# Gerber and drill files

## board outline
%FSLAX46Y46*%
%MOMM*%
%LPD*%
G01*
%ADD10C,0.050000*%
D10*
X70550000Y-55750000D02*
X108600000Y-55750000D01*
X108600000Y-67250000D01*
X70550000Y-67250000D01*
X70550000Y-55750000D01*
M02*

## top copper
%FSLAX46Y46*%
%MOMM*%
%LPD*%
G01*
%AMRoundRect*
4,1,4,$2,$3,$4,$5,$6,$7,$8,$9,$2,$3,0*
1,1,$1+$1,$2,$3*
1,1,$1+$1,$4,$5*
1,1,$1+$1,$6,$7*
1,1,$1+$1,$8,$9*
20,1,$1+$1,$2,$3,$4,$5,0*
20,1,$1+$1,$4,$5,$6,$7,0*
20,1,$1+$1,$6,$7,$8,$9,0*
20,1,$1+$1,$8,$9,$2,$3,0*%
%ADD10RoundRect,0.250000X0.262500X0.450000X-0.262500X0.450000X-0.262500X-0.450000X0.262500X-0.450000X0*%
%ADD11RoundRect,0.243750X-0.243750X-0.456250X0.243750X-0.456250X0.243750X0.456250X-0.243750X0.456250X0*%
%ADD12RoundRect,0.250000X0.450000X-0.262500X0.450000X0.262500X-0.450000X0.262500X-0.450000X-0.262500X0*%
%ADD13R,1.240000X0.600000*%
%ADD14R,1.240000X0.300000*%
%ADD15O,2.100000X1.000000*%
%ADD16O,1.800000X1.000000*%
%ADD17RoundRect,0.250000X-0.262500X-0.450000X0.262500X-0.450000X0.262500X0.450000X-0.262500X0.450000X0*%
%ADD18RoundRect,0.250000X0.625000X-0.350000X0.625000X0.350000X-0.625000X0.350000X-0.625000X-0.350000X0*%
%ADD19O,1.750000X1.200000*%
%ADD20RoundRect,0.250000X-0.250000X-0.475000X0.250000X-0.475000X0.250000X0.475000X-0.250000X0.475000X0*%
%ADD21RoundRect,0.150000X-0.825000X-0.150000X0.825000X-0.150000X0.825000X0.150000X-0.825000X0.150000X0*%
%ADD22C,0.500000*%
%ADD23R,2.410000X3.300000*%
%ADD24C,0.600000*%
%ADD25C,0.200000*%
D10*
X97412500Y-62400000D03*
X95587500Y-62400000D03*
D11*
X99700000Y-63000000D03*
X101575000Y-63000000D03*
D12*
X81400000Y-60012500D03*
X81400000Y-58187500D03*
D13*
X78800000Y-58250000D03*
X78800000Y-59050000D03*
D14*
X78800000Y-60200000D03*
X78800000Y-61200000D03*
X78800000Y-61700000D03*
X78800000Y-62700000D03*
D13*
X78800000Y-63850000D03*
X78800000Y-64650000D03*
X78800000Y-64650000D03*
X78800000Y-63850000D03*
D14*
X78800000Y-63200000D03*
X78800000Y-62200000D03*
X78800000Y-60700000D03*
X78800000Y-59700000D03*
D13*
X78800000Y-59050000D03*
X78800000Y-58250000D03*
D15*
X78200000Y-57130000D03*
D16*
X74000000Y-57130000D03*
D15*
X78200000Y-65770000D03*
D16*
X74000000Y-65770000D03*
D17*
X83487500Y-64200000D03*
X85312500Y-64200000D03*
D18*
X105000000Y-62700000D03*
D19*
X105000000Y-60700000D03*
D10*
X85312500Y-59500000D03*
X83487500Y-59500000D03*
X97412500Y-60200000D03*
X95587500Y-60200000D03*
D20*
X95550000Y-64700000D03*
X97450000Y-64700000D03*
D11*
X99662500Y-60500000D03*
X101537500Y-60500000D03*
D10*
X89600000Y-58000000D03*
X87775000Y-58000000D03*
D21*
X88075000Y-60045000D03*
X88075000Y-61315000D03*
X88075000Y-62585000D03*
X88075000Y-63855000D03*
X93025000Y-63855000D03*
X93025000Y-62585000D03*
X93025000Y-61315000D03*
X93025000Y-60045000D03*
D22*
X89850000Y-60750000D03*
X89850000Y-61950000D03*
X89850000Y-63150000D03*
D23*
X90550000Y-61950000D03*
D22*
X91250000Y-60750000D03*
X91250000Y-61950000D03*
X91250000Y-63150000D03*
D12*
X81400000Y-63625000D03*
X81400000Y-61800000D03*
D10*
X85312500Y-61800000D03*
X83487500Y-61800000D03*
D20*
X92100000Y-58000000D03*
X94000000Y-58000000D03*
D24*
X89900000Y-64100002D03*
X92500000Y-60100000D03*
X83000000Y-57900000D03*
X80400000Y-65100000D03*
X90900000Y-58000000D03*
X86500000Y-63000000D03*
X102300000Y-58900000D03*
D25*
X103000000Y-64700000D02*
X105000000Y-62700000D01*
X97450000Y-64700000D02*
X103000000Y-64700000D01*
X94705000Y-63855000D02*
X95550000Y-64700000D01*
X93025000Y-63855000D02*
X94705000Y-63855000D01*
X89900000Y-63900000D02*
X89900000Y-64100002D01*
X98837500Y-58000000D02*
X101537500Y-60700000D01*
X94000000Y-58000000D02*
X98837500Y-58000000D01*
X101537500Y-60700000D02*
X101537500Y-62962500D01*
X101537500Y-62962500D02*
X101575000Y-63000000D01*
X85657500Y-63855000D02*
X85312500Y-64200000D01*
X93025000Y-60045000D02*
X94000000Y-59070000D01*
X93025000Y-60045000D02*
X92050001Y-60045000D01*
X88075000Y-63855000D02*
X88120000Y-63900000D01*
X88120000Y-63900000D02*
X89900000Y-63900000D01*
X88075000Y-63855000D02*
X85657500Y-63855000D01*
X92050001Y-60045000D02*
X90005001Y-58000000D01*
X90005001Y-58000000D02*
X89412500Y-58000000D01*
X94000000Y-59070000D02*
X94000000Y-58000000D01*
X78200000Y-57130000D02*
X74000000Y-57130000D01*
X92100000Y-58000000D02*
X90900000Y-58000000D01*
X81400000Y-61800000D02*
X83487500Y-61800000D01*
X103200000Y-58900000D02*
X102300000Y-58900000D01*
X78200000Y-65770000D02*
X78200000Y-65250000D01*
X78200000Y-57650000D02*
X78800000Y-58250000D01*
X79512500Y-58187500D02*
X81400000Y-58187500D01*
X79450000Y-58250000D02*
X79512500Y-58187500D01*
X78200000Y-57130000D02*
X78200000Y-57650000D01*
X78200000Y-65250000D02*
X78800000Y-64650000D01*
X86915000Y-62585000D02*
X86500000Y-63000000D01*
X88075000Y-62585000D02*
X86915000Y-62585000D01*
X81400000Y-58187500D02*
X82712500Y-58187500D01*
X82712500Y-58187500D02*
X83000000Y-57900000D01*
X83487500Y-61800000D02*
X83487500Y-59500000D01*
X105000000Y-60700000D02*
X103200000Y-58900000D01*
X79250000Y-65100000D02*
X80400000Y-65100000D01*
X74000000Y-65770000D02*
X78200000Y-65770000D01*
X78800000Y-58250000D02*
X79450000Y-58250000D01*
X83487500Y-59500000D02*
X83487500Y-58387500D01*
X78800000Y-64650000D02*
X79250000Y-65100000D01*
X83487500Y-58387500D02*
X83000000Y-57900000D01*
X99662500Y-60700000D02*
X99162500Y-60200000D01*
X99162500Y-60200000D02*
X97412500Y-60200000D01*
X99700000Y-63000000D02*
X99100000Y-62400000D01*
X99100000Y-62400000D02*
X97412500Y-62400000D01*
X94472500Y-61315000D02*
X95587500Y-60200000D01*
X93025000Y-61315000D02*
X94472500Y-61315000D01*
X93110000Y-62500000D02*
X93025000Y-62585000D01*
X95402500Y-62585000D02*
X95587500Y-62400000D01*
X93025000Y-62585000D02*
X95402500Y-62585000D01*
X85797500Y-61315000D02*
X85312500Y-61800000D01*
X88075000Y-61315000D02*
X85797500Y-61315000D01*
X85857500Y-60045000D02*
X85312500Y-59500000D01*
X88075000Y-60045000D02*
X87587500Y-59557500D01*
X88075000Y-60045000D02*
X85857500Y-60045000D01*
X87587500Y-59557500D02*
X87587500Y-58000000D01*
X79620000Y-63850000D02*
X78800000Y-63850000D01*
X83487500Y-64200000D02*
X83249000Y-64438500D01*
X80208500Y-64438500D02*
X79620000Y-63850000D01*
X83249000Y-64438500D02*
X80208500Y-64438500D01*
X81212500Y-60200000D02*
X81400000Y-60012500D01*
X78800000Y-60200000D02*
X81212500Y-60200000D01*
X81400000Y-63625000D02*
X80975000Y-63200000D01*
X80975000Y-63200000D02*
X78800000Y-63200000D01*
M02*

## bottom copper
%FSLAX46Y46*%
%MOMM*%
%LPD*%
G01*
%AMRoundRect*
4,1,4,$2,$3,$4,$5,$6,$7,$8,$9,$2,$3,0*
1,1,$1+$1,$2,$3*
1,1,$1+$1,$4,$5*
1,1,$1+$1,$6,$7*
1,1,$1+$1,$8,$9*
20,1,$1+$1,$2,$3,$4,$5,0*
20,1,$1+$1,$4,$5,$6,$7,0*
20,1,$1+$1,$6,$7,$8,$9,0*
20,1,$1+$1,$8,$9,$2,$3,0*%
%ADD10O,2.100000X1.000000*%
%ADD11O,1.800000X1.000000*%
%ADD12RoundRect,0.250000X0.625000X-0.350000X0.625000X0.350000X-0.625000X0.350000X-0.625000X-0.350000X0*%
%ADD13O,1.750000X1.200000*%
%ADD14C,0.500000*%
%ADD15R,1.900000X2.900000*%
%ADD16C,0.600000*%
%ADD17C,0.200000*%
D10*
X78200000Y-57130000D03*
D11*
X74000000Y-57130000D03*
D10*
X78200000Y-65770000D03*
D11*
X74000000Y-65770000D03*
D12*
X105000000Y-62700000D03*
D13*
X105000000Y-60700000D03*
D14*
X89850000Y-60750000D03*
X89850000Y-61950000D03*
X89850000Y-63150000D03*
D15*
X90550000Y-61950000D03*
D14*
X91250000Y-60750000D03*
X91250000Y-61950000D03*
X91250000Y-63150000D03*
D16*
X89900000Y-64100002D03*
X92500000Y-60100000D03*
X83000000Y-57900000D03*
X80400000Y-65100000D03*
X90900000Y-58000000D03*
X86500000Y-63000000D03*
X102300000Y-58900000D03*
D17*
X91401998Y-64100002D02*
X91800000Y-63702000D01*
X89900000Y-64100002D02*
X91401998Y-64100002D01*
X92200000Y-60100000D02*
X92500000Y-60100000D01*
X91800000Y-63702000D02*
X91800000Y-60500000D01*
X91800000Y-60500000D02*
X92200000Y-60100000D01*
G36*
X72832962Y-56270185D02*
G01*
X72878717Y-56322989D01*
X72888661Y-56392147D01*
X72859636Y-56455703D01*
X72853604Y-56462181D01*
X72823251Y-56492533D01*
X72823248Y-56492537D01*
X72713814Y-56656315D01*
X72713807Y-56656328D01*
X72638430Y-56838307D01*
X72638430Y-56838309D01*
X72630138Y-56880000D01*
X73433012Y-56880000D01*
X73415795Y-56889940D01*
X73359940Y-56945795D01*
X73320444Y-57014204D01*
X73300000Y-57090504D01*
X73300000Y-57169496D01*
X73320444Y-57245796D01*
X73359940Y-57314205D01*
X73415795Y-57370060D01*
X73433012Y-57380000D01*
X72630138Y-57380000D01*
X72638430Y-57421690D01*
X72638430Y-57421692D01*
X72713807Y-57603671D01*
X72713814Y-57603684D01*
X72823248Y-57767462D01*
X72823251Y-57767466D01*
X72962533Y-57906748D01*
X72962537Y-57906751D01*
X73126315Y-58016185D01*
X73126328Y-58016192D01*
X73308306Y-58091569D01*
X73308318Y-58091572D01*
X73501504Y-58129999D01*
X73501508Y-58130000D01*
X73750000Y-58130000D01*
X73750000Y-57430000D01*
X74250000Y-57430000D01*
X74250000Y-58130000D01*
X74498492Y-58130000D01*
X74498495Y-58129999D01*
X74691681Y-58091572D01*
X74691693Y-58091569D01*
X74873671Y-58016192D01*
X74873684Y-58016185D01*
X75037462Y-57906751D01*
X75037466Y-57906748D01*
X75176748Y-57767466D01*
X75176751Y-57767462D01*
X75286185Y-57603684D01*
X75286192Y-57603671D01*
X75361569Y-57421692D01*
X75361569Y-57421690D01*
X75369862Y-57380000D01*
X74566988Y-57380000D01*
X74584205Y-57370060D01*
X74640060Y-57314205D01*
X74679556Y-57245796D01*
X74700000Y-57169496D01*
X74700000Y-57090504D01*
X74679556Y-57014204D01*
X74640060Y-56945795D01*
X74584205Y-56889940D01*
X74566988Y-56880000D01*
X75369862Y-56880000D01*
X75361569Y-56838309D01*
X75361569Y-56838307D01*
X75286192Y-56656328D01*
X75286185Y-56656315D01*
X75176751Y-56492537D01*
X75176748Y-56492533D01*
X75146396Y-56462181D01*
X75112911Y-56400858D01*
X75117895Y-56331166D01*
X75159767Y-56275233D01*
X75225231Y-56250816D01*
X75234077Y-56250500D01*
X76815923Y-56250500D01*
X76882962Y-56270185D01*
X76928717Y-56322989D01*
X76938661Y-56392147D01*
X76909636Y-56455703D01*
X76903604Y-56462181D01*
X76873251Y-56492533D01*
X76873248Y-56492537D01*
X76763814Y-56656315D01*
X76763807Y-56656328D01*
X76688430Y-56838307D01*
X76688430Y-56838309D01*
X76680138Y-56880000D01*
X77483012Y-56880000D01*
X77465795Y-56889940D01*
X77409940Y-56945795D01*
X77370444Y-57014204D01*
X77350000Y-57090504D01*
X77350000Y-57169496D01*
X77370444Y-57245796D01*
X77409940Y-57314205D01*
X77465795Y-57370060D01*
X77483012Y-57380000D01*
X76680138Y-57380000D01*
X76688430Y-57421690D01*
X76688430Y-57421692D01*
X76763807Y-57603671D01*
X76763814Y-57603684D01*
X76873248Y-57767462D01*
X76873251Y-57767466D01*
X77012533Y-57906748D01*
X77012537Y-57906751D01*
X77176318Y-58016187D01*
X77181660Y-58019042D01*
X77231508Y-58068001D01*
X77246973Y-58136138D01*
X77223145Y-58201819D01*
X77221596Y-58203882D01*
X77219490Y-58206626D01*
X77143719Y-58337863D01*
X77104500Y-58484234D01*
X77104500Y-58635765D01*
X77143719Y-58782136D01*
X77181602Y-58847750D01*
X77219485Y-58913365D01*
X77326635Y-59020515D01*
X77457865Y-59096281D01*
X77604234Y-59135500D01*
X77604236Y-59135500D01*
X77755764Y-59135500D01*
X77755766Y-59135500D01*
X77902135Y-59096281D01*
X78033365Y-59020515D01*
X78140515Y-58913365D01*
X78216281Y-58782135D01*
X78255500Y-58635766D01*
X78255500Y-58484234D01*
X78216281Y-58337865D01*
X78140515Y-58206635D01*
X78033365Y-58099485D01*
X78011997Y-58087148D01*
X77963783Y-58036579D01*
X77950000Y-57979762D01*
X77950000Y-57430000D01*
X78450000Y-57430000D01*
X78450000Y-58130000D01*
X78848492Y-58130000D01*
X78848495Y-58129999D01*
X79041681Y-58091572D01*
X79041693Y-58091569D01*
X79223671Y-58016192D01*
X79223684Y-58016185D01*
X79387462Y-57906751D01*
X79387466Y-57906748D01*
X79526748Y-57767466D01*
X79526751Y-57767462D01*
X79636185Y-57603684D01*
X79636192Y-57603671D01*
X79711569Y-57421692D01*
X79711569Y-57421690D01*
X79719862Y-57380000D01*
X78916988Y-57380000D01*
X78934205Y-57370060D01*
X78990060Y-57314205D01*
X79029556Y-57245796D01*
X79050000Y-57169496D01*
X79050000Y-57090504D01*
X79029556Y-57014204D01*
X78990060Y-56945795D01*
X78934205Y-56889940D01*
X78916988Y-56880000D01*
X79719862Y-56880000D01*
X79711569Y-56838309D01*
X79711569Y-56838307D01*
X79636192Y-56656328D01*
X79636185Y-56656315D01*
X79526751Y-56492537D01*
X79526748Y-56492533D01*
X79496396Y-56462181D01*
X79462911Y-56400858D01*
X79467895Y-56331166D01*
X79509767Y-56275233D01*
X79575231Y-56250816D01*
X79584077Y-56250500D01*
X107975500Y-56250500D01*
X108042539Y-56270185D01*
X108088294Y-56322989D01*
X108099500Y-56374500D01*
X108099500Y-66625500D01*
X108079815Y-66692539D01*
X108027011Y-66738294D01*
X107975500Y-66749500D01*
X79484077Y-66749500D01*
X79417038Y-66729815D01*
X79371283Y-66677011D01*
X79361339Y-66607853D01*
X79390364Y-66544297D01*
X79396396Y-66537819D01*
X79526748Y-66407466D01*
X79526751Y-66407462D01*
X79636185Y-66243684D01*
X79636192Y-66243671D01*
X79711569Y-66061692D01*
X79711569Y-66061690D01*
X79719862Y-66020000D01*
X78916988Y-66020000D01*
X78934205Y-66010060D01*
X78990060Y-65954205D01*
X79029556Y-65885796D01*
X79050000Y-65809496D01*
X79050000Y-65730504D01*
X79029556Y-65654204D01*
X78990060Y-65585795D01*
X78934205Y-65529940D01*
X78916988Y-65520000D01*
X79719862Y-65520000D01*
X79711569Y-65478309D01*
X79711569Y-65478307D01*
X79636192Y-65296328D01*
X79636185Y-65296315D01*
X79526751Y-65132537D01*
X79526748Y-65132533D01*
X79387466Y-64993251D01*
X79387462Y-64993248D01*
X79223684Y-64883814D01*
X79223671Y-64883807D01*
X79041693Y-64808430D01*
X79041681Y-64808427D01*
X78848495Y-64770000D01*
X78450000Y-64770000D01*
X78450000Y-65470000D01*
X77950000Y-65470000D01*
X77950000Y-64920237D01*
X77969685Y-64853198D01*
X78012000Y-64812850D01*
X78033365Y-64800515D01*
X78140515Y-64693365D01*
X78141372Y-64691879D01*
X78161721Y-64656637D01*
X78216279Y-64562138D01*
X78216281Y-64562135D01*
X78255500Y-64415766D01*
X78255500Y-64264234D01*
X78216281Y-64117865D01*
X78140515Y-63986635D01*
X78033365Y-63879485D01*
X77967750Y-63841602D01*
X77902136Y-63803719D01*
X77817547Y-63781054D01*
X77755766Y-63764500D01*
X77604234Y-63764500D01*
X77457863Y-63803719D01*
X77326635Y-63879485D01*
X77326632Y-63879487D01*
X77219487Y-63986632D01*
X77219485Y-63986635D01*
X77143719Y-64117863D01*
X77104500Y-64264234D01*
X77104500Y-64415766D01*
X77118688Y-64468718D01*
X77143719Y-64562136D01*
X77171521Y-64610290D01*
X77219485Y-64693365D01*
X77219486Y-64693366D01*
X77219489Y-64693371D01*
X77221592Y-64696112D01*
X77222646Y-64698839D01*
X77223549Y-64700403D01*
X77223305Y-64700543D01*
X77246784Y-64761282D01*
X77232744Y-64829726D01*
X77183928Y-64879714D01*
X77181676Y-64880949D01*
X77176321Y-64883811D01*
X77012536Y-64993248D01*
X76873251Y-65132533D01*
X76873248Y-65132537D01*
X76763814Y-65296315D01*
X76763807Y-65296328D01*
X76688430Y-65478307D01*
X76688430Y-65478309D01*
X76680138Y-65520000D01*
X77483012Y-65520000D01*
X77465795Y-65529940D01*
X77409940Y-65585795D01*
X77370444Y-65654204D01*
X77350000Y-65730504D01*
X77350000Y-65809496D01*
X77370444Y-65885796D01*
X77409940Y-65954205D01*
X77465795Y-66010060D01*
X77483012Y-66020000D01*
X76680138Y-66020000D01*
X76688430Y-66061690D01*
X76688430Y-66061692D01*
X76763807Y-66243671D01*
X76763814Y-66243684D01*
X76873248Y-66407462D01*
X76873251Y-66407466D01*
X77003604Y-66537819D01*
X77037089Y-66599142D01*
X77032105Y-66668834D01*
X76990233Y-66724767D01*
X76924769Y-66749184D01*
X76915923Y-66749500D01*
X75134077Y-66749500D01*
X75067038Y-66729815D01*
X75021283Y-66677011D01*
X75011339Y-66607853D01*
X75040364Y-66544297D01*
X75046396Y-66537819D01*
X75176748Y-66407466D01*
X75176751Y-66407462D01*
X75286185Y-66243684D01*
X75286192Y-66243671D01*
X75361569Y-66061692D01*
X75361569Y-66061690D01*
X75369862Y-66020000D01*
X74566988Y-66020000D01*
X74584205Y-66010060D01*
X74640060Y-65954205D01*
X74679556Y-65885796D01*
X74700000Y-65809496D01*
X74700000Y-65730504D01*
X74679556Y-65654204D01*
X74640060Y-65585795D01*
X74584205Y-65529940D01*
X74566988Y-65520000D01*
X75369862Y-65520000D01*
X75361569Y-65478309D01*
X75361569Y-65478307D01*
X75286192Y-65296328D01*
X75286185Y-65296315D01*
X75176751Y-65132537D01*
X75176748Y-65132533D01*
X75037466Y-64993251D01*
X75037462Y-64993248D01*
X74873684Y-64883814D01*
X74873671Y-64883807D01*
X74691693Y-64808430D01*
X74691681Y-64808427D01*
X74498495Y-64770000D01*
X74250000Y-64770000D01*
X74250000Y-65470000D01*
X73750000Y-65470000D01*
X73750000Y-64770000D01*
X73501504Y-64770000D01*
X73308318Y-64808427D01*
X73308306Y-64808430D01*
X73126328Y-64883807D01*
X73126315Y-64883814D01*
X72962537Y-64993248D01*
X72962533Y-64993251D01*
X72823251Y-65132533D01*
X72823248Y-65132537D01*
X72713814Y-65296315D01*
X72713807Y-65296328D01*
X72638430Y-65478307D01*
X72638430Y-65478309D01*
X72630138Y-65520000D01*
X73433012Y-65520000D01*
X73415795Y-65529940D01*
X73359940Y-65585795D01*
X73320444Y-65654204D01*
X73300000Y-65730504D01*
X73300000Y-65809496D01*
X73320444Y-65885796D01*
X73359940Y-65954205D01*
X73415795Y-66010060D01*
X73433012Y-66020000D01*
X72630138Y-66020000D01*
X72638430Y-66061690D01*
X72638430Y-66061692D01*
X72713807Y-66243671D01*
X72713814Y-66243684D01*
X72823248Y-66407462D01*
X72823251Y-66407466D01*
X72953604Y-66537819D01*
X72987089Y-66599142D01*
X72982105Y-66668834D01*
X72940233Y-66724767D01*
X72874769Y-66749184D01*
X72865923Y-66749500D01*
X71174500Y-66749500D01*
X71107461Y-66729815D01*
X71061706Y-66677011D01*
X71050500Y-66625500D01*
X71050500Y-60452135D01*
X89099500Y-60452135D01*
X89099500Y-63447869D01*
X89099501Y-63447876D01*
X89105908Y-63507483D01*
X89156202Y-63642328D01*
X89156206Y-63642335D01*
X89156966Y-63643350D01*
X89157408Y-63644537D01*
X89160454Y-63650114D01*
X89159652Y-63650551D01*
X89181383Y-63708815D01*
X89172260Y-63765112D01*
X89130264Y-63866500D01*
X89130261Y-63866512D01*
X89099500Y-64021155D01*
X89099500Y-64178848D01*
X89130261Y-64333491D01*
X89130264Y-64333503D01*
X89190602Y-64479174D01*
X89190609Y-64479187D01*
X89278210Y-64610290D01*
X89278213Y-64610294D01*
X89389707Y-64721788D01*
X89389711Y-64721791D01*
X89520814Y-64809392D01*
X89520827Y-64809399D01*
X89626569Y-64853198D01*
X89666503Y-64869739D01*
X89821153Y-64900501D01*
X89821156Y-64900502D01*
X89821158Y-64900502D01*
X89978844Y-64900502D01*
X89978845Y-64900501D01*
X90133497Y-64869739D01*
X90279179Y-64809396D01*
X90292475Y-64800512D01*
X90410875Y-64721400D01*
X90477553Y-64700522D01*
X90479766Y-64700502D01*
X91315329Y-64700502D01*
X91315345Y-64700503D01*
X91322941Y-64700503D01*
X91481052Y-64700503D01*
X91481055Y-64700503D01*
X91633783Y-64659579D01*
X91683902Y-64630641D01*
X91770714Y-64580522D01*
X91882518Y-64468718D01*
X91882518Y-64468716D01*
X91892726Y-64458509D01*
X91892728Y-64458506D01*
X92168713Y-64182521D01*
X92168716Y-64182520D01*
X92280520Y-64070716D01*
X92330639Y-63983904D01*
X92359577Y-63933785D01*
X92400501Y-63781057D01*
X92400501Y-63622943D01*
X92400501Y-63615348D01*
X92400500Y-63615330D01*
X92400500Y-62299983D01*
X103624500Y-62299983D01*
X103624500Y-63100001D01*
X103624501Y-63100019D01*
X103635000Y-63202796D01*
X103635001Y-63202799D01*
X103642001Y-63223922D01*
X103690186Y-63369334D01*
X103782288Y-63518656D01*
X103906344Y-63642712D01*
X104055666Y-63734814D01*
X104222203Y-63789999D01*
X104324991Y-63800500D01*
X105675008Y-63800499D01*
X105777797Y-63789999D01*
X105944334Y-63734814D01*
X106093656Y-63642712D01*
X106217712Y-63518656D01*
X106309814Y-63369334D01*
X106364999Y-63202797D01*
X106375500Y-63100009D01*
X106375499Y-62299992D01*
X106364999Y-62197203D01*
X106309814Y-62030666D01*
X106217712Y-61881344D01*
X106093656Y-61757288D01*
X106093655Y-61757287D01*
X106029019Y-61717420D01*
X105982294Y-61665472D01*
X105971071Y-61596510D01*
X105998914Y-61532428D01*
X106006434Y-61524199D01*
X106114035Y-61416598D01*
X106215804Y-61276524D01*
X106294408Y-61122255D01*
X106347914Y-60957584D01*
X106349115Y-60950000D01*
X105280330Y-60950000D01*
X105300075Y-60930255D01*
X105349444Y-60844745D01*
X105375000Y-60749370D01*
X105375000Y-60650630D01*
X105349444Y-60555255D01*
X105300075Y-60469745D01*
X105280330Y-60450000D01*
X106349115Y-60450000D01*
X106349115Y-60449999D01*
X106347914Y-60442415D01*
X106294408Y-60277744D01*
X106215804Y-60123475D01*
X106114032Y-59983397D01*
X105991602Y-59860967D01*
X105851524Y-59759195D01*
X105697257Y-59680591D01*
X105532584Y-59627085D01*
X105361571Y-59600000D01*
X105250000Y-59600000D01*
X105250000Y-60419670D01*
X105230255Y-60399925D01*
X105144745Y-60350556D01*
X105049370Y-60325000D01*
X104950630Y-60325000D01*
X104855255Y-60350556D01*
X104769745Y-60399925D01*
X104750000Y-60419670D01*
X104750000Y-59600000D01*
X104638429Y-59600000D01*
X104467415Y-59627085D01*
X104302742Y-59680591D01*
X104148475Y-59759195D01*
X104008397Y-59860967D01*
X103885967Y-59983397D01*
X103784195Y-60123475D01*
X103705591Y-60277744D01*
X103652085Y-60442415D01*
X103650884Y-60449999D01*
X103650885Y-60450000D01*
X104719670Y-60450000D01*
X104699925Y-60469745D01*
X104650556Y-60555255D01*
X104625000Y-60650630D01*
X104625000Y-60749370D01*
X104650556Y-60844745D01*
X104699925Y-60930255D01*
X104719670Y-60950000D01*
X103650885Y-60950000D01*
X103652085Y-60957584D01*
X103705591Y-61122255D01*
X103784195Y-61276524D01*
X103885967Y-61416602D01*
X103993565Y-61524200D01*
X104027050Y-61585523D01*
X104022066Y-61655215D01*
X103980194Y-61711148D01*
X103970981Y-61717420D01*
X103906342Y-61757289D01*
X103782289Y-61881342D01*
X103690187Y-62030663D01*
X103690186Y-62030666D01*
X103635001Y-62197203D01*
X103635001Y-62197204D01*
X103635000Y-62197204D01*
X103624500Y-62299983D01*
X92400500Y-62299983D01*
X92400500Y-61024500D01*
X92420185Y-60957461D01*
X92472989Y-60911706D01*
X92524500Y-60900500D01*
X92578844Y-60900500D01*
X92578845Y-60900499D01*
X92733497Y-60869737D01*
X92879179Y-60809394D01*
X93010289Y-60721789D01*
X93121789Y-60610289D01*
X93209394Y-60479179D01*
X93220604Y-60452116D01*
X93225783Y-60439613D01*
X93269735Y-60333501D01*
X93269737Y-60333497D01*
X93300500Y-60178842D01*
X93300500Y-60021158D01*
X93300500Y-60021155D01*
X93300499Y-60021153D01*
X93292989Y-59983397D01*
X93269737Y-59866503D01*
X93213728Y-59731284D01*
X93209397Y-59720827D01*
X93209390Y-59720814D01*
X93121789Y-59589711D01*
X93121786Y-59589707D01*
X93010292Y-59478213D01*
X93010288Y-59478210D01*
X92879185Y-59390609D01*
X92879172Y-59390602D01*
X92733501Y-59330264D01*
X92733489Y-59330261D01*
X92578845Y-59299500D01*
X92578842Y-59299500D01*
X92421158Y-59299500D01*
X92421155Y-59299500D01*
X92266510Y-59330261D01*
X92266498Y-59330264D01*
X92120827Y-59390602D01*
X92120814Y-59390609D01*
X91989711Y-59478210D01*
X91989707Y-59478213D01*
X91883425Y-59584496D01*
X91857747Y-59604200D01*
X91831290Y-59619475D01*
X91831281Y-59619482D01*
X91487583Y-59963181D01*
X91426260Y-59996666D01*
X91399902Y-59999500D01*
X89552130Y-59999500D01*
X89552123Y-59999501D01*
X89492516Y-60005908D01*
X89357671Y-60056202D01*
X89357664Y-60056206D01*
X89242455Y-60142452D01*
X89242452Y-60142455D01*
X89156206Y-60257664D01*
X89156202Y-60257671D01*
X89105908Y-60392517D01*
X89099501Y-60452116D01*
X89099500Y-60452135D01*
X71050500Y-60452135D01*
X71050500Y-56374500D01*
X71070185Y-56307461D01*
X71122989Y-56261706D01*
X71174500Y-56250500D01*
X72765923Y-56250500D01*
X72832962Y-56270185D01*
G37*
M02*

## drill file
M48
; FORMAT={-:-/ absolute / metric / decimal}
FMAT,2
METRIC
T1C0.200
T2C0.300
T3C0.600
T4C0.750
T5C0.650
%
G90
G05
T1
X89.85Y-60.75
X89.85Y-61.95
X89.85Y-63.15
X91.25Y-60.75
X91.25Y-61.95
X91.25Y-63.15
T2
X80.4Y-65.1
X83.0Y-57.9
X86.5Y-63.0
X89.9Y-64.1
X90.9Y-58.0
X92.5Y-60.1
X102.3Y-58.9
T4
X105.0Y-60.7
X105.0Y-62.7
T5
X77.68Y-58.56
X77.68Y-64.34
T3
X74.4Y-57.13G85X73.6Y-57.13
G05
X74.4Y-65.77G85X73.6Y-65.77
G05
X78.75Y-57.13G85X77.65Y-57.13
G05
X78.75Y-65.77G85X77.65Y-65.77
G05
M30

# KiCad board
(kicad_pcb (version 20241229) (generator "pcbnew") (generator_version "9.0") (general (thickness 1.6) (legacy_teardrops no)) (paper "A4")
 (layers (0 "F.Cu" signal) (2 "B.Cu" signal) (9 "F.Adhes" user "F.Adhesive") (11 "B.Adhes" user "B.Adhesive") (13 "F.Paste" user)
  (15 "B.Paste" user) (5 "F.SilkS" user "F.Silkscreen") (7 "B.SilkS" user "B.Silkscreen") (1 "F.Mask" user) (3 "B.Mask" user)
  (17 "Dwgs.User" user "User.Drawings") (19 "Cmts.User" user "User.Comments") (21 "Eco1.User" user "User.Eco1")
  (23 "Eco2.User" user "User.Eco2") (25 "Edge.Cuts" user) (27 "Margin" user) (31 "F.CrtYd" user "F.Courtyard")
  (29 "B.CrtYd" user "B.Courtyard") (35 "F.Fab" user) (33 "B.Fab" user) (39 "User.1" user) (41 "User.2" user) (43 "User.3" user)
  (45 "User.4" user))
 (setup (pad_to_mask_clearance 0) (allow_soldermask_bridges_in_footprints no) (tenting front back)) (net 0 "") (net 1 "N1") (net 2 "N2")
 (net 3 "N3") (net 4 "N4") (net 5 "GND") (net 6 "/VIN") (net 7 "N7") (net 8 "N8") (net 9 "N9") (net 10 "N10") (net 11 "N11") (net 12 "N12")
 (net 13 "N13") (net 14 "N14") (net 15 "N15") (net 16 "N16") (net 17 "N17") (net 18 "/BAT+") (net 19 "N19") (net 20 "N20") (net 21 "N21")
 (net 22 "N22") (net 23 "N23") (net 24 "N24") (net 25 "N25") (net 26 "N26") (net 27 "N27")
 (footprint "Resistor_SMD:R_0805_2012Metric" (layer "F.Cu") (at 96.5 62.4 180)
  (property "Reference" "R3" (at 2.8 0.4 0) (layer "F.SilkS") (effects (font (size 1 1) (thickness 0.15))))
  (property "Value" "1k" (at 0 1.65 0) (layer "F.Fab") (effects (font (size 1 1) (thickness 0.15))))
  (pad "1" smd roundrect (at -0.9125 0 180) (size 1.025 1.4) (layers "F.Cu" "F.Mask" "F.Paste") (roundrect_rratio 0.243902) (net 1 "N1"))
  (pad "2" smd roundrect (at 0.9125 0 180) (size 1.025 1.4) (layers "F.Cu" "F.Mask" "F.Paste") (roundrect_rratio 0.243902) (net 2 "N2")))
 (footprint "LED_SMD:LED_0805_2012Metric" (layer "F.Cu") (at 100.6375 63)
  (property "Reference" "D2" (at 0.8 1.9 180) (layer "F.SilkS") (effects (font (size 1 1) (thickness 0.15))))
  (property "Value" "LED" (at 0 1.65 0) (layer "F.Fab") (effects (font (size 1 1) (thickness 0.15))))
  (pad "1" smd roundrect (at -0.9375 0) (size 0.975 1.4) (layers "F.Cu" "F.Mask" "F.Paste") (roundrect_rratio 0.25) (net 1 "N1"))
  (pad "2" smd roundrect (at 0.9375 0) (size 0.975 1.4) (layers "F.Cu" "F.Mask" "F.Paste") (roundrect_rratio 0.25) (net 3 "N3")))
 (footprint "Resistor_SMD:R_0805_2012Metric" (layer "F.Cu") (at 81.4 59.1 90)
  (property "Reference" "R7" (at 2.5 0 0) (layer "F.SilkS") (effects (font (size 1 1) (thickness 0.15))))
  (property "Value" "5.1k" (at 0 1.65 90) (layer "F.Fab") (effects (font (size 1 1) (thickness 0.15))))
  (pad "1" smd roundrect (at -0.9125 0 90) (size 1.025 1.4) (layers "F.Cu" "F.Mask" "F.Paste") (roundrect_rratio 0.243902) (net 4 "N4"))
  (pad "2" smd roundrect (at 0.9125 0 90) (size 1.025 1.4) (layers "F.Cu" "F.Mask" "F.Paste") (roundrect_rratio 0.243902) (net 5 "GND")))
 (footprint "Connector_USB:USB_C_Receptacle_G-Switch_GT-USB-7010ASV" (layer "F.Cu") (at 75.075 61.45 -90)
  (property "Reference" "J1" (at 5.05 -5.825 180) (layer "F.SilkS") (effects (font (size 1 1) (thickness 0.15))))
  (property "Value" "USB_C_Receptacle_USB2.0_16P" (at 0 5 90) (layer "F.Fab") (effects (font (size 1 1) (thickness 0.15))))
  (pad "" np_thru_hole circle (at -2.89 -2.605 270) (size 0.65 0.65) (drill 0.65) (layers "*.Cu" "*.Mask"))
  (pad "" np_thru_hole circle (at 2.89 -2.605 270) (size 0.65 0.65) (drill 0.65) (layers "*.Cu" "*.Mask"))
  (pad "A1" smd rect (at -3.2 -3.725 270) (size 0.6 1.24) (layers "F.Cu" "F.Mask" "F.Paste") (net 5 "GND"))
  (pad "A4" smd rect (at -2.4 -3.725 270) (size 0.6 1.24) (layers "F.Cu" "F.Mask" "F.Paste") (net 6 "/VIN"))
  (pad "A5" smd rect (at -1.25 -3.725 270) (size 0.3 1.24) (layers "F.Cu" "F.Mask" "F.Paste") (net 4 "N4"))
  (pad "A6" smd rect (at -0.25 -3.725 270) (size 0.3 1.24) (layers "F.Cu" "F.Mask" "F.Paste") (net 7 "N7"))
  (pad "A7" smd rect (at 0.25 -3.725 270) (size 0.3 1.24) (layers "F.Cu" "F.Mask" "F.Paste") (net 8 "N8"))
  (pad "A8" smd rect (at 1.25 -3.725 270) (size 0.3 1.24) (layers "F.Cu" "F.Mask" "F.Paste") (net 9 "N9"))
  (pad "A9" smd rect (at 2.4 -3.725 270) (size 0.6 1.24) (layers "F.Cu" "F.Mask" "F.Paste") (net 6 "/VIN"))
  (pad "A12" smd rect (at 3.2 -3.725 270) (size 0.6 1.24) (layers "F.Cu" "F.Mask" "F.Paste") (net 5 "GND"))
  (pad "B1" smd rect (at 3.2 -3.725 270) (size 0.6 1.24) (layers "F.Cu" "F.Mask" "F.Paste") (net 5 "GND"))
  (pad "B4" smd rect (at 2.4 -3.725 270) (size 0.6 1.24) (layers "F.Cu" "F.Mask" "F.Paste") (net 6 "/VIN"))
  (pad "B5" smd rect (at 1.75 -3.725 270) (size 0.3 1.24) (layers "F.Cu" "F.Mask" "F.Paste") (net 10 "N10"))
  (pad "B6" smd rect (at 0.75 -3.725 270) (size 0.3 1.24) (layers "F.Cu" "F.Mask" "F.Paste") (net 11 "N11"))
  (pad "B7" smd rect (at -0.75 -3.725 270) (size 0.3 1.24) (layers "F.Cu" "F.Mask" "F.Paste") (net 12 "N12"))
  (pad "B8" smd rect (at -1.75 -3.725 270) (size 0.3 1.24) (layers "F.Cu" "F.Mask" "F.Paste") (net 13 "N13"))
  (pad "B9" smd rect (at -2.4 -3.725 270) (size 0.6 1.24) (layers "F.Cu" "F.Mask" "F.Paste") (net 6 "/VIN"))
  (pad "B12" smd rect (at -3.2 -3.725 270) (size 0.6 1.24) (layers "F.Cu" "F.Mask" "F.Paste") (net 5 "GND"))
  (pad "S1" thru_hole oval (at -4.32 -3.125 270) (size 1 2.1) (drill oval 0.6 1.7) (layers "*.Cu" "*.Mask") (remove_unused_layers no)
   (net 5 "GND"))
  (pad "S1" thru_hole oval (at -4.32 1.075 270) (size 1 1.8) (drill oval 0.6 1.4) (layers "*.Cu" "*.Mask") (remove_unused_layers no)
   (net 5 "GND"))
  (pad "S1" thru_hole oval (at 4.32 -3.125 270) (size 1 2.1) (drill oval 0.6 1.7) (layers "*.Cu" "*.Mask") (remove_unused_layers no)
   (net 5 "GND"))
  (pad "S1" thru_hole oval (at 4.32 1.075 270) (size 1 1.8) (drill oval 0.6 1.4) (layers "*.Cu" "*.Mask") (remove_unused_layers no)
   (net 5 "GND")))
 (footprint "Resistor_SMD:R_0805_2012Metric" (layer "F.Cu") (at 84.4 64.2)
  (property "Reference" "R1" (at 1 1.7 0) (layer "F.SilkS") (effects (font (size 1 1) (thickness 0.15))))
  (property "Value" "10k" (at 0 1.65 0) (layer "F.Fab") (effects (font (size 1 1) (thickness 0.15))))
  (pad "1" smd roundrect (at -0.9125 0) (size 1.025 1.4) (layers "F.Cu" "F.Mask" "F.Paste") (roundrect_rratio 0.243902) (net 6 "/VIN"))
  (pad "2" smd roundrect (at 0.9125 0) (size 1.025 1.4) (layers "F.Cu" "F.Mask" "F.Paste") (roundrect_rratio 0.243902) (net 3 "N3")))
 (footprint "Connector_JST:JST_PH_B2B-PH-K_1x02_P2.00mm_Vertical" (layer "F.Cu") (at 105 62.7 90)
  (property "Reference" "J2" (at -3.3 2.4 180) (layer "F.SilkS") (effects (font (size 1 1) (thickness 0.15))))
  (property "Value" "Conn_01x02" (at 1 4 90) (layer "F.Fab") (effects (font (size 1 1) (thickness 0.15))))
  (pad "1" thru_hole roundrect (at 0 0 90) (size 1.2 1.75) (drill 0.75) (layers "*.Cu" "*.Mask") (remove_unused_layers no)
   (roundrect_rratio 0.208333) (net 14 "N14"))
  (pad "2" thru_hole oval (at 2 0 90) (size 1.2 1.75) (drill 0.75) (layers "*.Cu" "*.Mask") (remove_unused_layers no) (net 5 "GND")))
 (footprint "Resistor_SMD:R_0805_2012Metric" (layer "F.Cu") (at 84.4 59.5 180)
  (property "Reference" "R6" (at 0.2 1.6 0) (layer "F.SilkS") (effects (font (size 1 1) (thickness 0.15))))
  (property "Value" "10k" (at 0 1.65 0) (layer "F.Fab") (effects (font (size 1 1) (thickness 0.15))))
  (pad "1" smd roundrect (at -0.9125 0 180) (size 1.025 1.4) (layers "F.Cu" "F.Mask" "F.Paste") (roundrect_rratio 0.243902) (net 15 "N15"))
  (pad "2" smd roundrect (at 0.9125 0 180) (size 1.025 1.4) (layers "F.Cu" "F.Mask" "F.Paste") (roundrect_rratio 0.243902) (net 5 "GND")))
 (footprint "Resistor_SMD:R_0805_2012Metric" (layer "F.Cu") (at 96.5 60.2 180)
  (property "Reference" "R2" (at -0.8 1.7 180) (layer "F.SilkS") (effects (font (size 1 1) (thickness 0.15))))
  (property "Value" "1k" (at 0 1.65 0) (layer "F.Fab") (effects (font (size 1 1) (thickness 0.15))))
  (pad "1" smd roundrect (at -0.9125 0 180) (size 1.025 1.4) (layers "F.Cu" "F.Mask" "F.Paste") (roundrect_rratio 0.243902) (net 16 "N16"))
  (pad "2" smd roundrect (at 0.9125 0 180) (size 1.025 1.4) (layers "F.Cu" "F.Mask" "F.Paste") (roundrect_rratio 0.243902) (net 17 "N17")))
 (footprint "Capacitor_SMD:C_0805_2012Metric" (layer "F.Cu") (at 96.5 64.7)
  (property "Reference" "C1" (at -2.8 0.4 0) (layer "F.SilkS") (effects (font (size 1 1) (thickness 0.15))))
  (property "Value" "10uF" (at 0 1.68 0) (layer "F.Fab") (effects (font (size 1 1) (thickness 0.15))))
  (pad "1" smd roundrect (at -0.95 0) (size 1 1.45) (layers "F.Cu" "F.Mask" "F.Paste") (roundrect_rratio 0.25) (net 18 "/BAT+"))
  (pad "2" smd roundrect (at 0.95 0) (size 1 1.45) (layers "F.Cu" "F.Mask" "F.Paste") (roundrect_rratio 0.25) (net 14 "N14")))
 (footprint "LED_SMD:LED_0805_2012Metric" (layer "F.Cu") (at 100.6 60.5)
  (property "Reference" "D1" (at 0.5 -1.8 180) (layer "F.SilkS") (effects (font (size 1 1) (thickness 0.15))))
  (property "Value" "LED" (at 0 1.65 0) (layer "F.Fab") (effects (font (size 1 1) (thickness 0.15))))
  (pad "1" smd roundrect (at -0.9375 0) (size 0.975 1.4) (layers "F.Cu" "F.Mask" "F.Paste") (roundrect_rratio 0.25) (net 16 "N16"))
  (pad "2" smd roundrect (at 0.9375 0) (size 0.975 1.4) (layers "F.Cu" "F.Mask" "F.Paste") (roundrect_rratio 0.25) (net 3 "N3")))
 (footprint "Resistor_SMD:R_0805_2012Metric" (layer "F.Cu") (at 88.6875 58 180)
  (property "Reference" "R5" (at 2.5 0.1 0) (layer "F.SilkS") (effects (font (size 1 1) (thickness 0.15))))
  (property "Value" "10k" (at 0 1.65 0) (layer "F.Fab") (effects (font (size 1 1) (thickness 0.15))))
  (pad "1" smd roundrect (at -0.9125 0 180) (size 1.025 1.4) (layers "F.Cu" "F.Mask" "F.Paste") (roundrect_rratio 0.243902) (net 3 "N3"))
  (pad "2" smd roundrect (at 0.9125 0 180) (size 1.025 1.4) (layers "F.Cu" "F.Mask" "F.Paste") (roundrect_rratio 0.243902) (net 15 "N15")))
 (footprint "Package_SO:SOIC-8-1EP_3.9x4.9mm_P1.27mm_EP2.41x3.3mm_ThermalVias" (layer "F.Cu") (at 90.55 61.95)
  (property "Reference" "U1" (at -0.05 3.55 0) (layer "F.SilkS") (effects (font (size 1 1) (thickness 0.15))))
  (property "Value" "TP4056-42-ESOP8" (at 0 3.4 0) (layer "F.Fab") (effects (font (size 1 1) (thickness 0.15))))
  (pad "" smd roundrect (at -0.6 -0.825) (size 1.01 1.38) (layers "F.Paste") (roundrect_rratio 0.247525))
  (pad "" smd roundrect (at -0.6 0.825) (size 1.01 1.38) (layers "F.Paste") (roundrect_rratio 0.247525))
  (pad "" smd roundrect (at 0.6 -0.825) (size 1.01 1.38) (layers "F.Paste") (roundrect_rratio 0.247525))
  (pad "" smd roundrect (at 0.6 0.825) (size 1.01 1.38) (layers "F.Paste") (roundrect_rratio 0.247525))
  (pad "1" smd roundrect (at -2.475 -1.905) (size 1.95 0.6) (layers "F.Cu" "F.Mask" "F.Paste") (roundrect_rratio 0.25) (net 15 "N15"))
  (pad "2" smd roundrect (at -2.475 -0.635) (size 1.95 0.6) (layers "F.Cu" "F.Mask" "F.Paste") (roundrect_rratio 0.25) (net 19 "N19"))
  (pad "3" smd roundrect (at -2.475 0.635) (size 1.95 0.6) (layers "F.Cu" "F.Mask" "F.Paste") (roundrect_rratio 0.25) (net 5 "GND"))
  (pad "4" smd roundrect (at -2.475 1.905) (size 1.95 0.6) (layers "F.Cu" "F.Mask" "F.Paste") (roundrect_rratio 0.25) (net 3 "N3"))
  (pad "5" smd roundrect (at 2.475 1.905) (size 1.95 0.6) (layers "F.Cu" "F.Mask" "F.Paste") (roundrect_rratio 0.25) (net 18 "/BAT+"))
  (pad "6" smd roundrect (at 2.475 0.635) (size 1.95 0.6) (layers "F.Cu" "F.Mask" "F.Paste") (roundrect_rratio 0.25) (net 2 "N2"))
  (pad "7" smd roundrect (at 2.475 -0.635) (size 1.95 0.6) (layers "F.Cu" "F.Mask" "F.Paste") (roundrect_rratio 0.25) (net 17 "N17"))
  (pad "8" smd roundrect (at 2.475 -1.905) (size 1.95 0.6) (layers "F.Cu" "F.Mask" "F.Paste") (roundrect_rratio 0.25) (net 3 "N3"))
  (pad "9" thru_hole circle (at -0.7 -1.2) (size 0.5 0.5) (drill 0.2) (layers "*.Cu") (remove_unused_layers no) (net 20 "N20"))
  (pad "9" thru_hole circle (at -0.7 0) (size 0.5 0.5) (drill 0.2) (layers "*.Cu") (remove_unused_layers no) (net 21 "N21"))
  (pad "9" thru_hole circle (at -0.7 1.2) (size 0.5 0.5) (drill 0.2) (layers "*.Cu") (remove_unused_layers no) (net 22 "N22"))
  (pad "9" smd rect (at 0 0) (size 1.9 2.9) (layers "B.Cu") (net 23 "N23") (zone_connect 2))
  (pad "9" smd rect (at 0 0) (size 2.41 3.3) (layers "F.Cu" "F.Mask") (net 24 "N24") (zone_connect 2))
  (pad "9" thru_hole circle (at 0.7 -1.2) (size 0.5 0.5) (drill 0.2) (layers "*.Cu") (remove_unused_layers no) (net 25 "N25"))
  (pad "9" thru_hole circle (at 0.7 0) (size 0.5 0.5) (drill 0.2) (layers "*.Cu") (remove_unused_layers no) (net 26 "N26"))
  (pad "9" thru_hole circle (at 0.7 1.2) (size 0.5 0.5) (drill 0.2) (layers "*.Cu") (remove_unused_layers no) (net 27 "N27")))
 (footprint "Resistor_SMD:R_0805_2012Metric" (layer "F.Cu") (at 81.4 62.7125 90)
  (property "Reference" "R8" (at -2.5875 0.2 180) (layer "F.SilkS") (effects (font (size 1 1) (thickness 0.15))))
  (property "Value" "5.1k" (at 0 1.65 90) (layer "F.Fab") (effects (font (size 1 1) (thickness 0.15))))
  (pad "1" smd roundrect (at -0.9125 0 90) (size 1.025 1.4) (layers "F.Cu" "F.Mask" "F.Paste") (roundrect_rratio 0.243902) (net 10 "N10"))
  (pad "2" smd roundrect (at 0.9125 0 90) (size 1.025 1.4) (layers "F.Cu" "F.Mask" "F.Paste") (roundrect_rratio 0.243902) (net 5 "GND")))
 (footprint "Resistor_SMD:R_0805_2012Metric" (layer "F.Cu") (at 84.4 61.8 180)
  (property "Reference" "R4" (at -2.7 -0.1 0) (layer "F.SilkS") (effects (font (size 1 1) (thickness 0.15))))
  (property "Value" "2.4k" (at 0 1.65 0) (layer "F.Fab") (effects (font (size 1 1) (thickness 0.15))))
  (pad "1" smd roundrect (at -0.9125 0 180) (size 1.025 1.4) (layers "F.Cu" "F.Mask" "F.Paste") (roundrect_rratio 0.243902) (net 19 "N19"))
  (pad "2" smd roundrect (at 0.9125 0 180) (size 1.025 1.4) (layers "F.Cu" "F.Mask" "F.Paste") (roundrect_rratio 0.243902) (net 5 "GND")))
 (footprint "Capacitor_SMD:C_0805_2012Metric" (layer "F.Cu") (at 93.05 58)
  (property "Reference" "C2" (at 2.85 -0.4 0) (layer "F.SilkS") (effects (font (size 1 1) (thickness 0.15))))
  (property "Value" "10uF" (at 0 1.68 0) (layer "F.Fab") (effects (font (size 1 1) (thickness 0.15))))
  (pad "1" smd roundrect (at -0.95 0) (size 1 1.45) (layers "F.Cu" "F.Mask" "F.Paste") (roundrect_rratio 0.25) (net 5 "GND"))
  (pad "2" smd roundrect (at 0.95 0) (size 1 1.45) (layers "F.Cu" "F.Mask" "F.Paste") (roundrect_rratio 0.25) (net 3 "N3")))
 (gr_rect (start 70.55 55.75) (end 108.6 67.25) (stroke (width 0.05) (type default)) (fill no) (layer "Edge.Cuts"))
 (segment (start 103 64.7) (end 105 62.7) (width 0.2) (layer "F.Cu") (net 14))
 (segment (start 97.45 64.7) (end 103 64.7) (width 0.2) (layer "F.Cu") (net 14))
 (segment (start 94.705 63.855) (end 95.55 64.7) (width 0.2) (layer "F.Cu") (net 18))
 (segment (start 93.025 63.855) (end 94.705 63.855) (width 0.2) (layer "F.Cu") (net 18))
 (segment (start 89.9 63.9) (end 89.9 64.100002) (width 0.2) (layer "F.Cu") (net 3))
 (segment (start 98.8375 58) (end 101.5375 60.7) (width 0.2) (layer "F.Cu") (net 3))
 (segment (start 94 58) (end 98.8375 58) (width 0.2) (layer "F.Cu") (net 3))
 (segment (start 101.5375 60.7) (end 101.5375 62.9625) (width 0.2) (layer "F.Cu") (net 3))
 (segment (start 101.5375 62.9625) (end 101.575 63) (width 0.2) (layer "F.Cu") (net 3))
 (segment (start 85.6575 63.855) (end 85.3125 64.2) (width 0.2) (layer "F.Cu") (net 3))
 (segment (start 93.025 60.045) (end 94 59.07) (width 0.2) (layer "F.Cu") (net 3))
 (segment (start 93.025 60.045) (end 92.050001 60.045) (width 0.2) (layer "F.Cu") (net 3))
 (segment (start 88.075 63.855) (end 88.12 63.9) (width 0.2) (layer "F.Cu") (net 3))
 (segment (start 88.12 63.9) (end 89.9 63.9) (width 0.2) (layer "F.Cu") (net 3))
 (segment (start 88.075 63.855) (end 85.6575 63.855) (width 0.2) (layer "F.Cu") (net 3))
 (segment (start 92.050001 60.045) (end 90.005001 58) (width 0.2) (layer "F.Cu") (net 3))
 (segment (start 90.005001 58) (end 89.4125 58) (width 0.2) (layer "F.Cu") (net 3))
 (segment (start 94 59.07) (end 94 58) (width 0.2) (layer "F.Cu") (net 3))
 (via (at 89.9 64.100002) (size 0.6) (drill 0.3) (layers "F.Cu" "B.Cu") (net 3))
 (via (at 92.5 60.1) (size 0.6) (drill 0.3) (layers "F.Cu" "B.Cu") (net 3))
 (segment (start 91.401998 64.100002) (end 91.8 63.702) (width 0.2) (layer "B.Cu") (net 3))
 (segment (start 89.9 64.100002) (end 91.401998 64.100002) (width 0.2) (layer "B.Cu") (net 3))
 (segment (start 92.2 60.1) (end 92.5 60.1) (width 0.2) (layer "B.Cu") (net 3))
 (segment (start 91.8 63.702) (end 91.8 60.5) (width 0.2) (layer "B.Cu") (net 3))
 (segment (start 91.8 60.5) (end 92.2 60.1) (width 0.2) (layer "B.Cu") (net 3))
 (segment (start 78.2 57.13) (end 74 57.13) (width 0.2) (layer "F.Cu") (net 5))
 (segment (start 92.1 58) (end 90.9 58) (width 0.2) (layer "F.Cu") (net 5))
 (segment (start 81.4 61.8) (end 83.4875 61.8) (width 0.2) (layer "F.Cu") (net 5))
 (segment (start 103.2 58.9) (end 102.3 58.9) (width 0.2) (layer "F.Cu") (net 5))
 (segment (start 78.2 65.77) (end 78.2 65.25) (width 0.2) (layer "F.Cu") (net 5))
 (segment (start 78.2 57.65) (end 78.8 58.25) (width 0.2) (layer "F.Cu") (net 5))
 (segment (start 79.5125 58.1875) (end 81.4 58.1875) (width 0.2) (layer "F.Cu") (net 5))
 (segment (start 79.45 58.25) (end 79.5125 58.1875) (width 0.2) (layer "F.Cu") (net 5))
 (segment (start 78.2 57.13) (end 78.2 57.65) (width 0.2) (layer "F.Cu") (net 5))
 (segment (start 78.2 65.25) (end 78.8 64.65) (width 0.2) (layer "F.Cu") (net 5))
 (segment (start 86.915 62.585) (end 86.5 63) (width 0.2) (layer "F.Cu") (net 5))
 (segment (start 88.075 62.585) (end 86.915 62.585) (width 0.2) (layer "F.Cu") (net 5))
 (segment (start 81.4 58.1875) (end 82.7125 58.1875) (width 0.2) (layer "F.Cu") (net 5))
 (segment (start 82.7125 58.1875) (end 83 57.9) (width 0.2) (layer "F.Cu") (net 5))
 (segment (start 83.4875 61.8) (end 83.4875 59.5) (width 0.2) (layer "F.Cu") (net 5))
 (segment (start 105 60.7) (end 103.2 58.9) (width 0.2) (layer "F.Cu") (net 5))
 (segment (start 79.25 65.1) (end 80.4 65.1) (width 0.2) (layer "F.Cu") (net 5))
 (segment (start 74 65.77) (end 78.2 65.77) (width 0.2) (layer "F.Cu") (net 5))
 (segment (start 78.8 58.25) (end 79.45 58.25) (width 0.2) (layer "F.Cu") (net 5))
 (segment (start 83.4875 59.5) (end 83.4875 58.3875) (width 0.2) (layer "F.Cu") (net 5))
 (segment (start 78.8 64.65) (end 79.25 65.1) (width 0.2) (layer "F.Cu") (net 5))
 (segment (start 83.4875 58.3875) (end 83 57.9) (width 0.2) (layer "F.Cu") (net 5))
 (via (at 83 57.9) (size 0.6) (drill 0.3) (layers "F.Cu" "B.Cu") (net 5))
 (via (at 80.4 65.1) (size 0.6) (drill 0.3) (layers "F.Cu" "B.Cu") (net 5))
 (via (at 90.9 58) (size 0.6) (drill 0.3) (layers "F.Cu" "B.Cu") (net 5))
 (via (at 86.5 63) (size 0.6) (drill 0.3) (layers "F.Cu" "B.Cu") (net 5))
 (via (at 102.3 58.9) (size 0.6) (drill 0.3) (layers "F.Cu" "B.Cu") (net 5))
 (segment (start 99.6625 60.7) (end 99.1625 60.2) (width 0.2) (layer "F.Cu") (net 16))
 (segment (start 99.1625 60.2) (end 97.4125 60.2) (width 0.2) (layer "F.Cu") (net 16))
 (segment (start 99.7 63) (end 99.1 62.4) (width 0.2) (layer "F.Cu") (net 1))
 (segment (start 99.1 62.4) (end 97.4125 62.4) (width 0.2) (layer "F.Cu") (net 1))
 (segment (start 94.4725 61.315) (end 95.5875 60.2) (width 0.2) (layer "F.Cu") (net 17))
 (segment (start 93.025 61.315) (end 94.4725 61.315) (width 0.2) (layer "F.Cu") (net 17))
 (segment (start 93.11 62.5) (end 93.025 62.585) (width 0.2) (layer "F.Cu") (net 2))
 (segment (start 95.4025 62.585) (end 95.5875 62.4) (width 0.2) (layer "F.Cu") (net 2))
 (segment (start 93.025 62.585) (end 95.4025 62.585) (width 0.2) (layer "F.Cu") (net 2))
 (segment (start 85.7975 61.315) (end 85.3125 61.8) (width 0.2) (layer "F.Cu") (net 19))
 (segment (start 88.075 61.315) (end 85.7975 61.315) (width 0.2) (layer "F.Cu") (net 19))
 (segment (start 85.8575 60.045) (end 85.3125 59.5) (width 0.2) (layer "F.Cu") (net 15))
 (segment (start 88.075 60.045) (end 87.5875 59.5575) (width 0.2) (layer "F.Cu") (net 15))
 (segment (start 88.075 60.045) (end 85.8575 60.045) (width 0.2) (layer "F.Cu") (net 15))
 (segment (start 87.5875 59.5575) (end 87.5875 58) (width 0.2) (layer "F.Cu") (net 15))
 (segment (start 79.62 63.85) (end 78.8 63.85) (width 0.2) (layer "F.Cu") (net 6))
 (segment (start 83.4875 64.2) (end 83.249 64.4385) (width 0.2) (layer "F.Cu") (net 6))
 (segment (start 80.2085 64.4385) (end 79.62 63.85) (width 0.2) (layer "F.Cu") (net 6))
 (segment (start 83.249 64.4385) (end 80.2085 64.4385) (width 0.2) (layer "F.Cu") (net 6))
 (segment (start 81.2125 60.2) (end 81.4 60.0125) (width 0.2) (layer "F.Cu") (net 4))
 (segment (start 78.8 60.2) (end 81.2125 60.2) (width 0.2) (layer "F.Cu") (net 4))
 (segment (start 81.4 63.625) (end 80.975 63.2) (width 0.2) (layer "F.Cu") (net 10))
 (segment (start 80.975 63.2) (end 78.8 63.2) (width 0.2) (layer "F.Cu") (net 10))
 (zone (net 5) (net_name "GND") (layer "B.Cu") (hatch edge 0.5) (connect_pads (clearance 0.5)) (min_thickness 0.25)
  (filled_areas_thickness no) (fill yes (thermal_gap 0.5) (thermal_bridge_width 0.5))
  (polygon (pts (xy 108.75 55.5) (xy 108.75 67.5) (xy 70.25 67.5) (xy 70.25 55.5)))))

